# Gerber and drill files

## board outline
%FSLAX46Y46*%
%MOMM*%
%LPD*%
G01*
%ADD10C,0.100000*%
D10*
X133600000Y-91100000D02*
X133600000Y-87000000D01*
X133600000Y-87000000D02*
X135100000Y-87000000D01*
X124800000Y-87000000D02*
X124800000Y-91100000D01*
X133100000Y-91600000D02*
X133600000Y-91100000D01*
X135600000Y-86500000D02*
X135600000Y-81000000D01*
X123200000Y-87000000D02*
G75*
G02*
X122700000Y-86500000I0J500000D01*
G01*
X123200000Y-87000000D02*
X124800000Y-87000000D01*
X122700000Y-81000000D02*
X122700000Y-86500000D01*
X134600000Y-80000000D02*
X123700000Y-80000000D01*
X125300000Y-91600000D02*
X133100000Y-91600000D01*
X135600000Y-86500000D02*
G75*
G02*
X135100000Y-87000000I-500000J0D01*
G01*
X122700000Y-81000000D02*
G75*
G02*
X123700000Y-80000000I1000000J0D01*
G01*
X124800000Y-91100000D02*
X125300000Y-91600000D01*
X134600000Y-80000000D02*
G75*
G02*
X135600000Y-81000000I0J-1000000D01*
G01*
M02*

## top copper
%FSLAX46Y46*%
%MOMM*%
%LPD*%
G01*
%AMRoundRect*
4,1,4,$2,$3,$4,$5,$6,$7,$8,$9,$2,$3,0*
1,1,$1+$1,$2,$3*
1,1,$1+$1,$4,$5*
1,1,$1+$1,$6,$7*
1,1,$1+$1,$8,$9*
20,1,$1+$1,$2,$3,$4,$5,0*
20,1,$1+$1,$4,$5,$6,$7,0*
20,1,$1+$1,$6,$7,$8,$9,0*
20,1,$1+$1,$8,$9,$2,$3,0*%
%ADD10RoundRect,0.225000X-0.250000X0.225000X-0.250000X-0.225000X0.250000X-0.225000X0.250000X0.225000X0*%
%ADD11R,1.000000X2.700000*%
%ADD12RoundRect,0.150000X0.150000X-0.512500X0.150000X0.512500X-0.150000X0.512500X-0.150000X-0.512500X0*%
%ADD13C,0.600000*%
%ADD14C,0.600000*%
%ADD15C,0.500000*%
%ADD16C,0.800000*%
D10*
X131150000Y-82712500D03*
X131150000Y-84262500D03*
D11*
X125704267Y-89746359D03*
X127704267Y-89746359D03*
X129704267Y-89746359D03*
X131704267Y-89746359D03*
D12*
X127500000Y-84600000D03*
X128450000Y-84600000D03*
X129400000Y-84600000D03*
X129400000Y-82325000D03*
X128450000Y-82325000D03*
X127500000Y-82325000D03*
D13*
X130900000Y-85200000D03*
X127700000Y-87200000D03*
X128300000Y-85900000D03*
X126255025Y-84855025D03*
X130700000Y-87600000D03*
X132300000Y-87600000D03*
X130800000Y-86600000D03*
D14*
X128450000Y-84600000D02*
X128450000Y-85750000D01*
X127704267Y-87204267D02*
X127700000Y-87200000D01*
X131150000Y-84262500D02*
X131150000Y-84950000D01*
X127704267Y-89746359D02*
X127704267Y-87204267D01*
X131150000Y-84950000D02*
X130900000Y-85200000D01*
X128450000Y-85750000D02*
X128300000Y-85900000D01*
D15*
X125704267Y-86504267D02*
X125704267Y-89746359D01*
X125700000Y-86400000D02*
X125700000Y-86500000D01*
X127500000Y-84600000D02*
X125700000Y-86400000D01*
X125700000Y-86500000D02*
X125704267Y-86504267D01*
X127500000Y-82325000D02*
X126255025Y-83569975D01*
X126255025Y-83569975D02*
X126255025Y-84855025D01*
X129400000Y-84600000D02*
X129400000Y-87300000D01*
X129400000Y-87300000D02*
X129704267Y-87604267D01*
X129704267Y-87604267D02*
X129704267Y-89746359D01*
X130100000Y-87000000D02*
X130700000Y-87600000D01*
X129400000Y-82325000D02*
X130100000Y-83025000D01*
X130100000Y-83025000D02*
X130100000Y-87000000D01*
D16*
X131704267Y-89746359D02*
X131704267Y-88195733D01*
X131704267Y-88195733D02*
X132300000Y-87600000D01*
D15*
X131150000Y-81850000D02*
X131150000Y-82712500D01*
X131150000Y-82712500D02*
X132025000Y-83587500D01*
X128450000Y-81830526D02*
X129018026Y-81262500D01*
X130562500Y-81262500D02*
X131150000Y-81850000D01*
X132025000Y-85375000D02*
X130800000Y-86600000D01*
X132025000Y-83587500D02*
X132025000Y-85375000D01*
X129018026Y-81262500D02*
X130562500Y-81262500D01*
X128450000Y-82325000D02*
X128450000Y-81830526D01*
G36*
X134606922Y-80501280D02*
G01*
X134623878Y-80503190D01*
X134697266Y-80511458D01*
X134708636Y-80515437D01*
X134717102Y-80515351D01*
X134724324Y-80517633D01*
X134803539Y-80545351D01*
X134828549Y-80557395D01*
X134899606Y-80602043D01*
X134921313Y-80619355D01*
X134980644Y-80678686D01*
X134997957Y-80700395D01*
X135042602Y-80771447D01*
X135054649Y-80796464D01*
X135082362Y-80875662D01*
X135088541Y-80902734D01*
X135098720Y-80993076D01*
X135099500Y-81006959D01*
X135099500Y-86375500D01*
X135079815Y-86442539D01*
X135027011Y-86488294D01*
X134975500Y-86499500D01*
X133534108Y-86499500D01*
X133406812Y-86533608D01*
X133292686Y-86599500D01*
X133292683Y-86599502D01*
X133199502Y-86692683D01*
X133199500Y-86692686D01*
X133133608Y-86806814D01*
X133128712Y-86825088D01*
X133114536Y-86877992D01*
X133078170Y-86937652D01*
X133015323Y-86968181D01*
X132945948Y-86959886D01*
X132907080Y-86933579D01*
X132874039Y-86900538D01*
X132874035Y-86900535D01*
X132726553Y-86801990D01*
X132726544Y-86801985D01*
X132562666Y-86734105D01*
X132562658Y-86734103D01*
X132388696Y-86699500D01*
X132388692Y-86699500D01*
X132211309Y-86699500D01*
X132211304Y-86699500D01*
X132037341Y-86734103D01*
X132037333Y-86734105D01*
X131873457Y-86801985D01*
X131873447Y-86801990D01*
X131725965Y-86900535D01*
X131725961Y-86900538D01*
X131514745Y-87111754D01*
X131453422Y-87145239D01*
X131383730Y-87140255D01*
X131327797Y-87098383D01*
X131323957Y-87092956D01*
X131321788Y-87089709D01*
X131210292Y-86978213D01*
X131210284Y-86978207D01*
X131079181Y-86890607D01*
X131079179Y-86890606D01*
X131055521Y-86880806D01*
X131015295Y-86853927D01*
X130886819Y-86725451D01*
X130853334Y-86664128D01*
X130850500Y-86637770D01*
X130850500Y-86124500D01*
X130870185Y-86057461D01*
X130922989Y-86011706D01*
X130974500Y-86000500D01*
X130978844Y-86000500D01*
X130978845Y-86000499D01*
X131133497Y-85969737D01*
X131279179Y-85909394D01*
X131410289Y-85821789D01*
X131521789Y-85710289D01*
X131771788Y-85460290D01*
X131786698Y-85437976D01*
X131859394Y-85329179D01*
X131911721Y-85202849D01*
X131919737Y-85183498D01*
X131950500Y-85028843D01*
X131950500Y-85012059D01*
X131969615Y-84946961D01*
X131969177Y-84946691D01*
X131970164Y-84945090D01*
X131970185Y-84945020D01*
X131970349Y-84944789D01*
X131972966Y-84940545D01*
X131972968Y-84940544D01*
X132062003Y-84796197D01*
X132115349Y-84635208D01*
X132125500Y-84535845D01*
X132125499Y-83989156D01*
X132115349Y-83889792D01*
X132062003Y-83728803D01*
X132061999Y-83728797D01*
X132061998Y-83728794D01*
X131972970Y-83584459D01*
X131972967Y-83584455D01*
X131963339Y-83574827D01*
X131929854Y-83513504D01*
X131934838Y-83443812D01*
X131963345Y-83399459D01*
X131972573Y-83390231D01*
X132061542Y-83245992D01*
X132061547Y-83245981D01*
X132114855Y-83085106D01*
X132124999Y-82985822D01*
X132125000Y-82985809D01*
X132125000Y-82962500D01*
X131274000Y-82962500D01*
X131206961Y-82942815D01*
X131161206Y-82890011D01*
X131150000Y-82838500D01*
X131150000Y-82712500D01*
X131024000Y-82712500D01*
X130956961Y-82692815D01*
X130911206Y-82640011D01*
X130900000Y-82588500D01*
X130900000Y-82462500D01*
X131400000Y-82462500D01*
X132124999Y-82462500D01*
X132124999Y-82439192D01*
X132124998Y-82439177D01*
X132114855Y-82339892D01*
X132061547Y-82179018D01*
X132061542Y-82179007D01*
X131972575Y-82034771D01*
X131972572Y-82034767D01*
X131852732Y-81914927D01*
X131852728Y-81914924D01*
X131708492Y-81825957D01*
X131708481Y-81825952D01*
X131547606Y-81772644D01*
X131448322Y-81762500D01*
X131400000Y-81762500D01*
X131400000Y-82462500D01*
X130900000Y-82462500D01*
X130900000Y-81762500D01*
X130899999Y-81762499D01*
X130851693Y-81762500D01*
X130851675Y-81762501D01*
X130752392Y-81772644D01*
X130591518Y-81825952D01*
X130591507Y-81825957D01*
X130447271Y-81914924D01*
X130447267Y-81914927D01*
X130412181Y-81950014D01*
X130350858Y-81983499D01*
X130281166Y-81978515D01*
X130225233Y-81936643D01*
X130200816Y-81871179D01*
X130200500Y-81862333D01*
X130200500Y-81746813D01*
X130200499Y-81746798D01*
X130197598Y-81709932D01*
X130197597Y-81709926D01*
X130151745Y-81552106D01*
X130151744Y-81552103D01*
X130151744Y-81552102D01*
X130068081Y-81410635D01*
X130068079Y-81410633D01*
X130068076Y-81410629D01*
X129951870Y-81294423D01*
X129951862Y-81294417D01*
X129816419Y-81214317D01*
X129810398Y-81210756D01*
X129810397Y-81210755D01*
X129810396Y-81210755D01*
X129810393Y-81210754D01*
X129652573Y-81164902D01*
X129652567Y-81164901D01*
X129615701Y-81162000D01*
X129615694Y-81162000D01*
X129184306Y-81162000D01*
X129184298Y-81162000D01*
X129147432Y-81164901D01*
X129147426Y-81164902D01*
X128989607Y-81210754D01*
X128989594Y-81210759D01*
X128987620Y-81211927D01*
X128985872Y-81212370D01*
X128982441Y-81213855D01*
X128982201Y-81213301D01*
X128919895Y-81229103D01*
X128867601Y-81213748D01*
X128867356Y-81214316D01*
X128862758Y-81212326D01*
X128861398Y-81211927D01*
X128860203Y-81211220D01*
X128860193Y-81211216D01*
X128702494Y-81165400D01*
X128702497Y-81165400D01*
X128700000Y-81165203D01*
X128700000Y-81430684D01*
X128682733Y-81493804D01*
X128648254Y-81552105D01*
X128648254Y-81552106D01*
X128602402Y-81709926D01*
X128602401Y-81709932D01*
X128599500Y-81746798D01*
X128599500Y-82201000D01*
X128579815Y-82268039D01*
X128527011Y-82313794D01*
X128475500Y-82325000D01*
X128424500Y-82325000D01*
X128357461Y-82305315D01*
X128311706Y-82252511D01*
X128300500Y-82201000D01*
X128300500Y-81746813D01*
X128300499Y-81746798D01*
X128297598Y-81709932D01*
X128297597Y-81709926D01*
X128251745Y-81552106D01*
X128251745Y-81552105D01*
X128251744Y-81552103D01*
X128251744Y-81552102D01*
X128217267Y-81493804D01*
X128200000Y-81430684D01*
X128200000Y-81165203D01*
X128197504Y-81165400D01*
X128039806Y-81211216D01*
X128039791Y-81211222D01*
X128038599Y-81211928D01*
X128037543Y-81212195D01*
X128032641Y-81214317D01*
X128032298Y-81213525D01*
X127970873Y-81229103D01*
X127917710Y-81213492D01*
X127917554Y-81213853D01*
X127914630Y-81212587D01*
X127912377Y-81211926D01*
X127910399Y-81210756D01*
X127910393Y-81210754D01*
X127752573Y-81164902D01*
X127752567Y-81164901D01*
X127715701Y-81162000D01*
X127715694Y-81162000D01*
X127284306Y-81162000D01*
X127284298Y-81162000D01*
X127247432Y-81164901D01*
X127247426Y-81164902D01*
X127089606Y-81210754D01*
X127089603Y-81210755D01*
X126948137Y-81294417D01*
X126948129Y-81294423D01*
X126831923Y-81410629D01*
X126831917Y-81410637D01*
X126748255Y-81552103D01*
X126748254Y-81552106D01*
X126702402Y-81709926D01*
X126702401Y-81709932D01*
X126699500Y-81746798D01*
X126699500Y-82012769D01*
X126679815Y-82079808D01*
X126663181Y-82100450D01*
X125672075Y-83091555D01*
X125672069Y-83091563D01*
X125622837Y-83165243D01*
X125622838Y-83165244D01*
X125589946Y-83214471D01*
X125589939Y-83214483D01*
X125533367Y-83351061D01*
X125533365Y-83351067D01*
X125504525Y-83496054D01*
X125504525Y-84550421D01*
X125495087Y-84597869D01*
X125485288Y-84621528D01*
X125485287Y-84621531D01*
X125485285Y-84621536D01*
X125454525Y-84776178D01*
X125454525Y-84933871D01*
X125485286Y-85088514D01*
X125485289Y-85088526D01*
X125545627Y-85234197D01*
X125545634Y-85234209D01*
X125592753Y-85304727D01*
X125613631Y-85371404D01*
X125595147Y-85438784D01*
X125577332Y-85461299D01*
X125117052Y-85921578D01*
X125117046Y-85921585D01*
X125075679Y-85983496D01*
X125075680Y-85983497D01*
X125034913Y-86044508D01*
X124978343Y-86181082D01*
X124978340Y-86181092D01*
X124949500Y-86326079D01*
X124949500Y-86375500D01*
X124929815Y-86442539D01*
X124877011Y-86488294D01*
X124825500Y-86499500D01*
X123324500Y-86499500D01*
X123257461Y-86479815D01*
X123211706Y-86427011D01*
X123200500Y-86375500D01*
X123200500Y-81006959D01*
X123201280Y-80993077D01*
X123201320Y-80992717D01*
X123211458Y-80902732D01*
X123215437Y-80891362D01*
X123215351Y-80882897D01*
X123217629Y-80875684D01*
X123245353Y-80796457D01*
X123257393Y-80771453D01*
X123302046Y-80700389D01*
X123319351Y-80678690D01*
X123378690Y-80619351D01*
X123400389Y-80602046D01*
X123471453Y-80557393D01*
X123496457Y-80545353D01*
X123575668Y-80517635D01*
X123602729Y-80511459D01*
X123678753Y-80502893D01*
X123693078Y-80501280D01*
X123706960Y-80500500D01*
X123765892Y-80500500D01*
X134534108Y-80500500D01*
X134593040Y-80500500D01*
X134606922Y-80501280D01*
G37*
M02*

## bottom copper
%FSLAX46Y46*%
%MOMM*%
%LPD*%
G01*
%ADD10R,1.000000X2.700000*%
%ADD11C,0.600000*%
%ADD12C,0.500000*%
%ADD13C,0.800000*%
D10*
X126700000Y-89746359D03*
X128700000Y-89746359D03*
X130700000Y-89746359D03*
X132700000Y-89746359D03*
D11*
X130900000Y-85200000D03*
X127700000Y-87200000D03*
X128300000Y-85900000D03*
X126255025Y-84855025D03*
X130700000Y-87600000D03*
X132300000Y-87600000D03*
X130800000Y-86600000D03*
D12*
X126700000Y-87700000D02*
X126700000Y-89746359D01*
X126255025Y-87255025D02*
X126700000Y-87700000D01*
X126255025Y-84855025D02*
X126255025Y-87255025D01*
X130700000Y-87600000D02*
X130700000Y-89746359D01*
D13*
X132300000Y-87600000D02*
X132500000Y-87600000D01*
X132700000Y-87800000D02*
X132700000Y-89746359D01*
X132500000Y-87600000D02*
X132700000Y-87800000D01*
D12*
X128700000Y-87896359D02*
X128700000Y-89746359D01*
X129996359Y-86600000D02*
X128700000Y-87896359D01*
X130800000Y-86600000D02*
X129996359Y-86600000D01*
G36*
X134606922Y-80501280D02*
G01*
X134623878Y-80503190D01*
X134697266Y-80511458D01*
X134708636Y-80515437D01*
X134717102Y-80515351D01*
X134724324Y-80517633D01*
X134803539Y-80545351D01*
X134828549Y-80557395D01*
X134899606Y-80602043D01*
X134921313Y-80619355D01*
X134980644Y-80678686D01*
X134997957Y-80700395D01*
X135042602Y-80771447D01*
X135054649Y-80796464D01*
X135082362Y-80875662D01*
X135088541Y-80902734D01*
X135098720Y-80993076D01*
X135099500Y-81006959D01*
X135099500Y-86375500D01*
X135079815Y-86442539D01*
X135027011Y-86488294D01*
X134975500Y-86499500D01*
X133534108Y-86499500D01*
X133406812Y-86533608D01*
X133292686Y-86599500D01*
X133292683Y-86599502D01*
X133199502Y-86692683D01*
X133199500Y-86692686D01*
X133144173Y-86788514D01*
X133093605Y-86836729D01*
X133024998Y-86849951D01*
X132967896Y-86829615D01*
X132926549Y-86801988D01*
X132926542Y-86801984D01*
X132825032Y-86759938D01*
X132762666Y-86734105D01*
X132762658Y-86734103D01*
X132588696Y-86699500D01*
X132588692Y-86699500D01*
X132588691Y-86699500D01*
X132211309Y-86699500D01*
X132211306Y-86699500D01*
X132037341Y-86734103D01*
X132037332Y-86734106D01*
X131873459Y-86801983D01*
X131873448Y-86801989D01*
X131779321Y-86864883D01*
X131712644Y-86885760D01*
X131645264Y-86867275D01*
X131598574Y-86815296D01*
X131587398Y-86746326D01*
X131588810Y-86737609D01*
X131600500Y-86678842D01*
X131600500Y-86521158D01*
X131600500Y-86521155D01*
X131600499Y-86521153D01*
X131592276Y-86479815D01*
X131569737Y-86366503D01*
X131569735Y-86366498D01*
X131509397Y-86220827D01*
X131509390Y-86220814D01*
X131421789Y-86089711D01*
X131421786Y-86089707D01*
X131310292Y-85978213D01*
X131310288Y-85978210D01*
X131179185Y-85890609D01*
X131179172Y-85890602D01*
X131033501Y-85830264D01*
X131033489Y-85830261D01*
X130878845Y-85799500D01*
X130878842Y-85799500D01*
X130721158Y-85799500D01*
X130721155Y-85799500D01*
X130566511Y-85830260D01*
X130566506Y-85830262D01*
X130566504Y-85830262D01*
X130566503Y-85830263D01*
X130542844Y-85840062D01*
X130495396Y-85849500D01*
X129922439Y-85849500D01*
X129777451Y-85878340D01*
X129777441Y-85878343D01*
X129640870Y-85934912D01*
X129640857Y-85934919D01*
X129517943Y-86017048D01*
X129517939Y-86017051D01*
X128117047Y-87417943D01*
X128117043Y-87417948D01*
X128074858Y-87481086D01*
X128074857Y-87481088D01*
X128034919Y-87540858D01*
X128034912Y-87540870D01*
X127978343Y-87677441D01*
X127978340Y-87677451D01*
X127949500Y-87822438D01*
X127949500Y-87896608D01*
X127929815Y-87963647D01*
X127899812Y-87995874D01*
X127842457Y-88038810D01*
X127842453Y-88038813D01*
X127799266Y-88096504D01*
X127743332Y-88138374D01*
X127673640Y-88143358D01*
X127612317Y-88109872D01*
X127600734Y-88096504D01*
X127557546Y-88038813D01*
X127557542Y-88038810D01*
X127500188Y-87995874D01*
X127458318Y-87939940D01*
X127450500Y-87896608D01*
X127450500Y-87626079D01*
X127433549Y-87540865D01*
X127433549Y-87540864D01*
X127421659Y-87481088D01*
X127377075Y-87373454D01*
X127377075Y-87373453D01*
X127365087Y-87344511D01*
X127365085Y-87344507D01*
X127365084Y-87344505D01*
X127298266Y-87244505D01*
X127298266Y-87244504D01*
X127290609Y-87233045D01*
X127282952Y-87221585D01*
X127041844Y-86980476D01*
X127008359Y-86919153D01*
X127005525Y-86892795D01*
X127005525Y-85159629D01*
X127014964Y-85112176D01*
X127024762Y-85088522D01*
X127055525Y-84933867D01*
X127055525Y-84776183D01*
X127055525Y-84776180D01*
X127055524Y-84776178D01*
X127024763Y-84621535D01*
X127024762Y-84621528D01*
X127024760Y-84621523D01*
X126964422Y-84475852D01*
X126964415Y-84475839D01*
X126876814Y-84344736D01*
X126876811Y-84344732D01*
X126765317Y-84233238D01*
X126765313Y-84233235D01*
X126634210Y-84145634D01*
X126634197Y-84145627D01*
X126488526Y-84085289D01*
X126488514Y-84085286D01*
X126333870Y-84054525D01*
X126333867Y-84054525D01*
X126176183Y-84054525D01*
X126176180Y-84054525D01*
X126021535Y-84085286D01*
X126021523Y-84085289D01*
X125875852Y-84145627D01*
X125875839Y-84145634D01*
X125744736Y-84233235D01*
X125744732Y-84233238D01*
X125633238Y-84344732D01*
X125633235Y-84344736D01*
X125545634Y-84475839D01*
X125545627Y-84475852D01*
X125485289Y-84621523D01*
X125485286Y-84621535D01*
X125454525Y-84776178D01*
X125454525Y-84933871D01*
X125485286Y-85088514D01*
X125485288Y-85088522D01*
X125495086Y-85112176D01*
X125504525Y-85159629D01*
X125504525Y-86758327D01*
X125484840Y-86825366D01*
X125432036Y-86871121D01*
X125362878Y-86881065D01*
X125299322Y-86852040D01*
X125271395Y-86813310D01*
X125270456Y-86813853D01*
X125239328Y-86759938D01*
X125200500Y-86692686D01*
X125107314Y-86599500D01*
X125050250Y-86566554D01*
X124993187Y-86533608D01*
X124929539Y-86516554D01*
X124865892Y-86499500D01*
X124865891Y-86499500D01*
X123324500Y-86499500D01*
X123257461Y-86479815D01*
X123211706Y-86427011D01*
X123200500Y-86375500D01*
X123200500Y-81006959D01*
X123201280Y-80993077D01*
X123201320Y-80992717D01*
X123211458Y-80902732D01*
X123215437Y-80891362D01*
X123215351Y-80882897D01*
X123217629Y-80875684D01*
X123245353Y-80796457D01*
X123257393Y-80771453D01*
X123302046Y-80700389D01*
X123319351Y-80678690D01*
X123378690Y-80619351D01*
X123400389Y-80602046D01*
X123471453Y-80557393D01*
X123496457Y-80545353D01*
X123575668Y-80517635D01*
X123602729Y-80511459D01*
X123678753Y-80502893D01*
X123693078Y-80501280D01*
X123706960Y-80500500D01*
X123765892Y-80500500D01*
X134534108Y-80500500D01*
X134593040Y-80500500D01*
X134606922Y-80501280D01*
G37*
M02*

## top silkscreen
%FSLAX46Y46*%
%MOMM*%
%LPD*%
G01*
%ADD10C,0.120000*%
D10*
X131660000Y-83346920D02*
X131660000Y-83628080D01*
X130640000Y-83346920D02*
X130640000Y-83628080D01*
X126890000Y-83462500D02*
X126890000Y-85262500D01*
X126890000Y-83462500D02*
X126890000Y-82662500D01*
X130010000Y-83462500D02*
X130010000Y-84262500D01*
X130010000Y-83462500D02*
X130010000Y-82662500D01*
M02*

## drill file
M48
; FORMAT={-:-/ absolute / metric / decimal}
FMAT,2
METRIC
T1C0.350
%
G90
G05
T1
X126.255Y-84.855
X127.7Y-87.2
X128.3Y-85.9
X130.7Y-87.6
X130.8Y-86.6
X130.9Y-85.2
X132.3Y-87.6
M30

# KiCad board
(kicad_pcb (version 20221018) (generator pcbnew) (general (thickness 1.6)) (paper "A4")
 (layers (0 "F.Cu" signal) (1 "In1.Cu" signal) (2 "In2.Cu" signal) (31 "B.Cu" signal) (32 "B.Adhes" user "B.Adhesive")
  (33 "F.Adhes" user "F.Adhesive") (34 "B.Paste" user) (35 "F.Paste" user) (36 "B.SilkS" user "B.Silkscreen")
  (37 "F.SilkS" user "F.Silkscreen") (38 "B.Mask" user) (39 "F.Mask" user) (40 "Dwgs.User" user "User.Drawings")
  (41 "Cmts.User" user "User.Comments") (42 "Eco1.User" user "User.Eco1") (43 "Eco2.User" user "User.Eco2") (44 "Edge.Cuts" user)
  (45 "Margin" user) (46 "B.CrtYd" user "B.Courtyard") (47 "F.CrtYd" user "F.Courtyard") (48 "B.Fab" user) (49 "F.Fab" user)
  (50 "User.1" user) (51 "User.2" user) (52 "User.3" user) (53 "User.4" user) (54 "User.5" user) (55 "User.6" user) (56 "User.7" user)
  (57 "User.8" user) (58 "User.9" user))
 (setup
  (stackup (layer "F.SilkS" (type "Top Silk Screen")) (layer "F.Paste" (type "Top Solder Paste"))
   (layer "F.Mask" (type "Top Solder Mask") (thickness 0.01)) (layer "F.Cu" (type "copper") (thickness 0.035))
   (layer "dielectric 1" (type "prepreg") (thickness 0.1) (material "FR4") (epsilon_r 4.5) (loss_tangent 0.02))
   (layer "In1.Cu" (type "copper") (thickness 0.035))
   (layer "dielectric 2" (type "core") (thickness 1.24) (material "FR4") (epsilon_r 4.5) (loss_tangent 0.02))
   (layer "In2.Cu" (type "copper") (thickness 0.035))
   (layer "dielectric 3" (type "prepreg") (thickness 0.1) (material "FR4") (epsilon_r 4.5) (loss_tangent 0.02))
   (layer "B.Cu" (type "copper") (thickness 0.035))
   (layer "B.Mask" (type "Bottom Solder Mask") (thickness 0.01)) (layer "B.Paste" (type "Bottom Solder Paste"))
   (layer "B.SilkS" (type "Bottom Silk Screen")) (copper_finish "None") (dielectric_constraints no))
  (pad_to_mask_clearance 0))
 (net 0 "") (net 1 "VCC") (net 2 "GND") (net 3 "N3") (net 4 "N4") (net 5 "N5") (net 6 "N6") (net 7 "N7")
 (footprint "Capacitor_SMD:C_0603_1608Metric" (layer "F.Cu") (at 131.15 83.4875 -90)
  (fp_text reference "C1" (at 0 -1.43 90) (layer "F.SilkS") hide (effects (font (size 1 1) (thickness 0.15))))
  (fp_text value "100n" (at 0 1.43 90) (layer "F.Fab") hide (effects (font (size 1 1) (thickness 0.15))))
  (fp_line (start -0.14058 -0.51) (end 0.14058 -0.51) (stroke (width 0.12) (type solid)) (layer "F.SilkS"))
  (fp_line (start -0.14058 0.51) (end 0.14058 0.51) (stroke (width 0.12) (type solid)) (layer "F.SilkS"))
  (pad "1" smd roundrect (at -0.775 0 270) (size 0.9 0.95) (layers "F.Cu" "F.Paste" "F.Mask") (roundrect_rratio 0.25) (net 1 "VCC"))
  (pad "2" smd roundrect (at 0.775 0 270) (size 0.9 0.95) (layers "F.Cu" "F.Paste" "F.Mask") (roundrect_rratio 0.25) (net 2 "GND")))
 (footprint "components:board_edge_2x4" (layer "F.Cu") (at 129.2 91.1)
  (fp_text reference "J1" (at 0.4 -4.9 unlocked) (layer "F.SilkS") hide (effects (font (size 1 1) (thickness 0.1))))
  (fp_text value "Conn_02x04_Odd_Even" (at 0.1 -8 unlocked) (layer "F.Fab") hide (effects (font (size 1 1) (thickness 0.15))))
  (pad "1" smd rect (at -3.495733 -1.353641) (size 1 2.7) (layers "F.Cu" "F.Paste" "F.Mask") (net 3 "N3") (thermal_bridge_angle 45))
  (pad "2" smd rect (at -2.5 -1.353641) (size 1 2.7) (layers "B.Cu" "B.Paste" "B.Mask") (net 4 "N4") (thermal_bridge_angle 45))
  (pad "3" smd rect (at -1.495733 -1.353641) (size 1 2.7) (layers "F.Cu" "F.Paste" "F.Mask") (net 2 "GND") (thermal_bridge_angle 45))
  (pad "4" smd rect (at -0.5 -1.353641) (size 1 2.7) (layers "B.Cu" "B.Paste" "B.Mask") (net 1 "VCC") (thermal_bridge_angle 45))
  (pad "5" smd rect (at 0.504267 -1.353641) (size 1 2.7) (layers "F.Cu" "F.Paste" "F.Mask") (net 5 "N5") (thermal_bridge_angle 45))
  (pad "6" smd rect (at 1.5 -1.353641) (size 1 2.7) (layers "B.Cu" "B.Paste" "B.Mask") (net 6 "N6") (thermal_bridge_angle 45))
  (pad "7" smd rect (at 2.504267 -1.353641) (size 1 2.7) (layers "F.Cu" "F.Paste" "F.Mask") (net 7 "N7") (thermal_bridge_angle 45))
  (pad "8" smd rect (at 3.5 -1.353641) (size 1 2.7) (layers "B.Cu" "B.Paste" "B.Mask") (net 7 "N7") (thermal_bridge_angle 45)))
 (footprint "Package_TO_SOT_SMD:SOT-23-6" (layer "F.Cu") (at 128.45 83.4625 90)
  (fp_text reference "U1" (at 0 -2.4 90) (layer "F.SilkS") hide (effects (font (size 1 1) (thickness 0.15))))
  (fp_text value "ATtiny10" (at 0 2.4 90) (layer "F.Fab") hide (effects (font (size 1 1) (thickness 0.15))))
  (fp_line (start 0 -1.56) (end -1.8 -1.56) (stroke (width 0.12) (type solid)) (layer "F.SilkS"))
  (fp_line (start 0 -1.56) (end 0.8 -1.56) (stroke (width 0.12) (type solid)) (layer "F.SilkS"))
  (fp_line (start 0 1.56) (end -0.8 1.56) (stroke (width 0.12) (type solid)) (layer "F.SilkS"))
  (fp_line (start 0 1.56) (end 0.8 1.56) (stroke (width 0.12) (type solid)) (layer "F.SilkS"))
  (pad "1" smd roundrect (at -1.1375 -0.95 90) (size 1.325 0.6) (layers "F.Cu" "F.Paste" "F.Mask") (roundrect_rratio 0.25) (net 3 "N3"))
  (pad "2" smd roundrect (at -1.1375 0 90) (size 1.325 0.6) (layers "F.Cu" "F.Paste" "F.Mask") (roundrect_rratio 0.25) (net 2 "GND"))
  (pad "3" smd roundrect (at -1.1375 0.95 90) (size 1.325 0.6) (layers "F.Cu" "F.Paste" "F.Mask") (roundrect_rratio 0.25) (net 5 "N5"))
  (pad "4" smd roundrect (at 1.1375 0.95 90) (size 1.325 0.6) (layers "F.Cu" "F.Paste" "F.Mask") (roundrect_rratio 0.25) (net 6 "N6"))
  (pad "5" smd roundrect (at 1.1375 0 90) (size 1.325 0.6) (layers "F.Cu" "F.Paste" "F.Mask") (roundrect_rratio 0.25) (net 1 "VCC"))
  (pad "6" smd roundrect (at 1.1375 -0.95 90) (size 1.325 0.6) (layers "F.Cu" "F.Paste" "F.Mask") (roundrect_rratio 0.25) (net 4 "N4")))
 (gr_line (start 133.6 91.1) (end 133.6 87) (stroke (width 0.1) (type default)) (layer "Edge.Cuts"))
 (gr_line (start 133.6 87) (end 135.1 87) (stroke (width 0.1) (type default)) (layer "Edge.Cuts"))
 (gr_line (start 124.8 87) (end 124.8 91.1) (stroke (width 0.1) (type default)) (layer "Edge.Cuts"))
 (gr_line (start 133.1 91.6) (end 133.6 91.1) (stroke (width 0.1) (type default)) (layer "Edge.Cuts"))
 (gr_line (start 135.6 86.5) (end 135.6 81) (stroke (width 0.1) (type default)) (layer "Edge.Cuts"))
 (gr_arc (start 123.2 87) (mid 122.846447 86.853553) (end 122.7 86.5) (stroke (width 0.1) (type default)) (layer "Edge.Cuts"))
 (gr_line (start 123.2 87) (end 124.8 87) (stroke (width 0.1) (type default)) (layer "Edge.Cuts"))
 (gr_line (start 122.7 81) (end 122.7 86.5) (stroke (width 0.1) (type default)) (layer "Edge.Cuts"))
 (gr_line (start 134.6 80) (end 123.7 80) (stroke (width 0.1) (type default)) (layer "Edge.Cuts"))
 (gr_line (start 125.3 91.6) (end 133.1 91.6) (stroke (width 0.1) (type default)) (layer "Edge.Cuts"))
 (gr_arc (start 135.6 86.5) (mid 135.453553 86.853553) (end 135.1 87) (stroke (width 0.1) (type default)) (layer "Edge.Cuts"))
 (gr_arc (start 122.7 81) (mid 122.992893 80.292893) (end 123.7 80) (stroke (width 0.1) (type default)) (layer "Edge.Cuts"))
 (gr_line (start 124.8 91.1) (end 125.3 91.6) (stroke (width 0.1) (type default)) (layer "Edge.Cuts"))
 (gr_arc (start 134.6 80) (mid 135.307107 80.292893) (end 135.6 81) (stroke (width 0.1) (type default)) (layer "Edge.Cuts"))
 (segment (start 128.45 84.6) (end 128.45 85.75) (width 0.6) (layer "F.Cu") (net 2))
 (segment (start 127.704267 87.204267) (end 127.7 87.2) (width 0.6) (layer "F.Cu") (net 2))
 (segment (start 131.15 84.2625) (end 131.15 84.95) (width 0.6) (layer "F.Cu") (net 2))
 (segment (start 127.704267 89.746359) (end 127.704267 87.204267) (width 0.6) (layer "F.Cu") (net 2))
 (segment (start 131.15 84.95) (end 130.9 85.2) (width 0.6) (layer "F.Cu") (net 2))
 (segment (start 128.45 85.75) (end 128.3 85.9) (width 0.6) (layer "F.Cu") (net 2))
 (via (at 130.9 85.2) (size 0.6) (drill 0.35) (layers "F.Cu" "B.Cu") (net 2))
 (via (at 127.7 87.2) (size 0.6) (drill 0.35) (layers "F.Cu" "B.Cu") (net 2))
 (via (at 128.3 85.9) (size 0.6) (drill 0.35) (layers "F.Cu" "B.Cu") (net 2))
 (segment (start 125.704267 86.504267) (end 125.704267 89.746359) (width 0.5) (layer "F.Cu") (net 3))
 (segment (start 125.7 86.4) (end 125.7 86.5) (width 0.5) (layer "F.Cu") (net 3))
 (segment (start 127.5 84.6) (end 125.7 86.4) (width 0.5) (layer "F.Cu") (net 3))
 (segment (start 125.7 86.5) (end 125.704267 86.504267) (width 0.5) (layer "F.Cu") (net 3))
 (segment (start 127.5 82.325) (end 126.255025 83.569975) (width 0.5) (layer "F.Cu") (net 4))
 (segment (start 126.255025 83.569975) (end 126.255025 84.855025) (width 0.5) (layer "F.Cu") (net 4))
 (via (at 126.255025 84.855025) (size 0.6) (drill 0.35) (layers "F.Cu" "B.Cu") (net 4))
 (segment (start 126.7 87.7) (end 126.7 89.746359) (width 0.5) (layer "B.Cu") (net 4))
 (segment (start 126.255025 87.255025) (end 126.7 87.7) (width 0.5) (layer "B.Cu") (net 4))
 (segment (start 126.255025 84.855025) (end 126.255025 87.255025) (width 0.5) (layer "B.Cu") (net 4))
 (segment (start 129.4 84.6) (end 129.4 87.3) (width 0.5) (layer "F.Cu") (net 5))
 (segment (start 129.4 87.3) (end 129.704267 87.604267) (width 0.5) (layer "F.Cu") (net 5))
 (segment (start 129.704267 87.604267) (end 129.704267 89.746359) (width 0.5) (layer "F.Cu") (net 5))
 (segment (start 130.1 87) (end 130.7 87.6) (width 0.5) (layer "F.Cu") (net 6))
 (segment (start 129.4 82.325) (end 130.1 83.025) (width 0.5) (layer "F.Cu") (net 6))
 (segment (start 130.1 83.025) (end 130.1 87) (width 0.5) (layer "F.Cu") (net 6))
 (via (at 130.7 87.6) (size 0.6) (drill 0.35) (layers "F.Cu" "B.Cu") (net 6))
 (segment (start 130.7 87.6) (end 130.7 89.746359) (width 0.5) (layer "B.Cu") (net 6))
 (segment (start 131.704267 89.746359) (end 131.704267 88.195733) (width 0.8) (layer "F.Cu") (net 7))
 (segment (start 131.704267 88.195733) (end 132.3 87.6) (width 0.8) (layer "F.Cu") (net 7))
 (via (at 132.3 87.6) (size 0.6) (drill 0.35) (layers "F.Cu" "B.Cu") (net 7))
 (segment (start 132.3 87.6) (end 132.5 87.6) (width 0.8) (layer "B.Cu") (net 7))
 (segment (start 132.7 87.8) (end 132.7 89.746359) (width 0.8) (layer "B.Cu") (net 7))
 (segment (start 132.5 87.6) (end 132.7 87.8) (width 0.8) (layer "B.Cu") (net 7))
 (segment (start 131.15 81.85) (end 131.15 82.7125) (width 0.5) (layer "F.Cu") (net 1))
 (segment (start 131.15 82.7125) (end 132.025 83.5875) (width 0.5) (layer "F.Cu") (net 1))
 (segment (start 128.45 81.830526) (end 129.018026 81.2625) (width 0.5) (layer "F.Cu") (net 1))
 (segment (start 130.5625 81.2625) (end 131.15 81.85) (width 0.5) (layer "F.Cu") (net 1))
 (segment (start 132.025 85.375) (end 130.8 86.6) (width 0.5) (layer "F.Cu") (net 1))
 (segment (start 132.025 83.5875) (end 132.025 85.375) (width 0.5) (layer "F.Cu") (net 1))
 (segment (start 129.018026 81.2625) (end 130.5625 81.2625) (width 0.5) (layer "F.Cu") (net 1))
 (segment (start 128.45 82.325) (end 128.45 81.830526) (width 0.5) (layer "F.Cu") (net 1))
 (via (at 130.8 86.6) (size 0.6) (drill 0.35) (layers "F.Cu" "B.Cu") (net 1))
 (segment (start 128.7 87.896359) (end 128.7 89.746359) (width 0.5) (layer "B.Cu") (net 1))
 (segment (start 129.996359 86.6) (end 128.7 87.896359) (width 0.5) (layer "B.Cu") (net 1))
 (segment (start 130.8 86.6) (end 129.996359 86.6) (width 0.5) (layer "B.Cu") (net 1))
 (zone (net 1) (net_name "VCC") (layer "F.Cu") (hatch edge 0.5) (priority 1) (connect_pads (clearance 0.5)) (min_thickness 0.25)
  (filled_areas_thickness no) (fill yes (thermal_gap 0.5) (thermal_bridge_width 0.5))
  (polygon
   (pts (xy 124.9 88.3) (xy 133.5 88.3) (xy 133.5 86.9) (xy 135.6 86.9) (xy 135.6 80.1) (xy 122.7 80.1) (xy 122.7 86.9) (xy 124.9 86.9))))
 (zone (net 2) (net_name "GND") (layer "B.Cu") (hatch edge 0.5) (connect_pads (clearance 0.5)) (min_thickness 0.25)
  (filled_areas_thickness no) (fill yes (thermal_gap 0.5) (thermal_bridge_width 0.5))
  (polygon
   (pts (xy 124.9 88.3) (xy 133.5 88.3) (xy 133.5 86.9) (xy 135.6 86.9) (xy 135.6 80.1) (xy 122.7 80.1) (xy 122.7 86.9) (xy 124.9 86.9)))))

